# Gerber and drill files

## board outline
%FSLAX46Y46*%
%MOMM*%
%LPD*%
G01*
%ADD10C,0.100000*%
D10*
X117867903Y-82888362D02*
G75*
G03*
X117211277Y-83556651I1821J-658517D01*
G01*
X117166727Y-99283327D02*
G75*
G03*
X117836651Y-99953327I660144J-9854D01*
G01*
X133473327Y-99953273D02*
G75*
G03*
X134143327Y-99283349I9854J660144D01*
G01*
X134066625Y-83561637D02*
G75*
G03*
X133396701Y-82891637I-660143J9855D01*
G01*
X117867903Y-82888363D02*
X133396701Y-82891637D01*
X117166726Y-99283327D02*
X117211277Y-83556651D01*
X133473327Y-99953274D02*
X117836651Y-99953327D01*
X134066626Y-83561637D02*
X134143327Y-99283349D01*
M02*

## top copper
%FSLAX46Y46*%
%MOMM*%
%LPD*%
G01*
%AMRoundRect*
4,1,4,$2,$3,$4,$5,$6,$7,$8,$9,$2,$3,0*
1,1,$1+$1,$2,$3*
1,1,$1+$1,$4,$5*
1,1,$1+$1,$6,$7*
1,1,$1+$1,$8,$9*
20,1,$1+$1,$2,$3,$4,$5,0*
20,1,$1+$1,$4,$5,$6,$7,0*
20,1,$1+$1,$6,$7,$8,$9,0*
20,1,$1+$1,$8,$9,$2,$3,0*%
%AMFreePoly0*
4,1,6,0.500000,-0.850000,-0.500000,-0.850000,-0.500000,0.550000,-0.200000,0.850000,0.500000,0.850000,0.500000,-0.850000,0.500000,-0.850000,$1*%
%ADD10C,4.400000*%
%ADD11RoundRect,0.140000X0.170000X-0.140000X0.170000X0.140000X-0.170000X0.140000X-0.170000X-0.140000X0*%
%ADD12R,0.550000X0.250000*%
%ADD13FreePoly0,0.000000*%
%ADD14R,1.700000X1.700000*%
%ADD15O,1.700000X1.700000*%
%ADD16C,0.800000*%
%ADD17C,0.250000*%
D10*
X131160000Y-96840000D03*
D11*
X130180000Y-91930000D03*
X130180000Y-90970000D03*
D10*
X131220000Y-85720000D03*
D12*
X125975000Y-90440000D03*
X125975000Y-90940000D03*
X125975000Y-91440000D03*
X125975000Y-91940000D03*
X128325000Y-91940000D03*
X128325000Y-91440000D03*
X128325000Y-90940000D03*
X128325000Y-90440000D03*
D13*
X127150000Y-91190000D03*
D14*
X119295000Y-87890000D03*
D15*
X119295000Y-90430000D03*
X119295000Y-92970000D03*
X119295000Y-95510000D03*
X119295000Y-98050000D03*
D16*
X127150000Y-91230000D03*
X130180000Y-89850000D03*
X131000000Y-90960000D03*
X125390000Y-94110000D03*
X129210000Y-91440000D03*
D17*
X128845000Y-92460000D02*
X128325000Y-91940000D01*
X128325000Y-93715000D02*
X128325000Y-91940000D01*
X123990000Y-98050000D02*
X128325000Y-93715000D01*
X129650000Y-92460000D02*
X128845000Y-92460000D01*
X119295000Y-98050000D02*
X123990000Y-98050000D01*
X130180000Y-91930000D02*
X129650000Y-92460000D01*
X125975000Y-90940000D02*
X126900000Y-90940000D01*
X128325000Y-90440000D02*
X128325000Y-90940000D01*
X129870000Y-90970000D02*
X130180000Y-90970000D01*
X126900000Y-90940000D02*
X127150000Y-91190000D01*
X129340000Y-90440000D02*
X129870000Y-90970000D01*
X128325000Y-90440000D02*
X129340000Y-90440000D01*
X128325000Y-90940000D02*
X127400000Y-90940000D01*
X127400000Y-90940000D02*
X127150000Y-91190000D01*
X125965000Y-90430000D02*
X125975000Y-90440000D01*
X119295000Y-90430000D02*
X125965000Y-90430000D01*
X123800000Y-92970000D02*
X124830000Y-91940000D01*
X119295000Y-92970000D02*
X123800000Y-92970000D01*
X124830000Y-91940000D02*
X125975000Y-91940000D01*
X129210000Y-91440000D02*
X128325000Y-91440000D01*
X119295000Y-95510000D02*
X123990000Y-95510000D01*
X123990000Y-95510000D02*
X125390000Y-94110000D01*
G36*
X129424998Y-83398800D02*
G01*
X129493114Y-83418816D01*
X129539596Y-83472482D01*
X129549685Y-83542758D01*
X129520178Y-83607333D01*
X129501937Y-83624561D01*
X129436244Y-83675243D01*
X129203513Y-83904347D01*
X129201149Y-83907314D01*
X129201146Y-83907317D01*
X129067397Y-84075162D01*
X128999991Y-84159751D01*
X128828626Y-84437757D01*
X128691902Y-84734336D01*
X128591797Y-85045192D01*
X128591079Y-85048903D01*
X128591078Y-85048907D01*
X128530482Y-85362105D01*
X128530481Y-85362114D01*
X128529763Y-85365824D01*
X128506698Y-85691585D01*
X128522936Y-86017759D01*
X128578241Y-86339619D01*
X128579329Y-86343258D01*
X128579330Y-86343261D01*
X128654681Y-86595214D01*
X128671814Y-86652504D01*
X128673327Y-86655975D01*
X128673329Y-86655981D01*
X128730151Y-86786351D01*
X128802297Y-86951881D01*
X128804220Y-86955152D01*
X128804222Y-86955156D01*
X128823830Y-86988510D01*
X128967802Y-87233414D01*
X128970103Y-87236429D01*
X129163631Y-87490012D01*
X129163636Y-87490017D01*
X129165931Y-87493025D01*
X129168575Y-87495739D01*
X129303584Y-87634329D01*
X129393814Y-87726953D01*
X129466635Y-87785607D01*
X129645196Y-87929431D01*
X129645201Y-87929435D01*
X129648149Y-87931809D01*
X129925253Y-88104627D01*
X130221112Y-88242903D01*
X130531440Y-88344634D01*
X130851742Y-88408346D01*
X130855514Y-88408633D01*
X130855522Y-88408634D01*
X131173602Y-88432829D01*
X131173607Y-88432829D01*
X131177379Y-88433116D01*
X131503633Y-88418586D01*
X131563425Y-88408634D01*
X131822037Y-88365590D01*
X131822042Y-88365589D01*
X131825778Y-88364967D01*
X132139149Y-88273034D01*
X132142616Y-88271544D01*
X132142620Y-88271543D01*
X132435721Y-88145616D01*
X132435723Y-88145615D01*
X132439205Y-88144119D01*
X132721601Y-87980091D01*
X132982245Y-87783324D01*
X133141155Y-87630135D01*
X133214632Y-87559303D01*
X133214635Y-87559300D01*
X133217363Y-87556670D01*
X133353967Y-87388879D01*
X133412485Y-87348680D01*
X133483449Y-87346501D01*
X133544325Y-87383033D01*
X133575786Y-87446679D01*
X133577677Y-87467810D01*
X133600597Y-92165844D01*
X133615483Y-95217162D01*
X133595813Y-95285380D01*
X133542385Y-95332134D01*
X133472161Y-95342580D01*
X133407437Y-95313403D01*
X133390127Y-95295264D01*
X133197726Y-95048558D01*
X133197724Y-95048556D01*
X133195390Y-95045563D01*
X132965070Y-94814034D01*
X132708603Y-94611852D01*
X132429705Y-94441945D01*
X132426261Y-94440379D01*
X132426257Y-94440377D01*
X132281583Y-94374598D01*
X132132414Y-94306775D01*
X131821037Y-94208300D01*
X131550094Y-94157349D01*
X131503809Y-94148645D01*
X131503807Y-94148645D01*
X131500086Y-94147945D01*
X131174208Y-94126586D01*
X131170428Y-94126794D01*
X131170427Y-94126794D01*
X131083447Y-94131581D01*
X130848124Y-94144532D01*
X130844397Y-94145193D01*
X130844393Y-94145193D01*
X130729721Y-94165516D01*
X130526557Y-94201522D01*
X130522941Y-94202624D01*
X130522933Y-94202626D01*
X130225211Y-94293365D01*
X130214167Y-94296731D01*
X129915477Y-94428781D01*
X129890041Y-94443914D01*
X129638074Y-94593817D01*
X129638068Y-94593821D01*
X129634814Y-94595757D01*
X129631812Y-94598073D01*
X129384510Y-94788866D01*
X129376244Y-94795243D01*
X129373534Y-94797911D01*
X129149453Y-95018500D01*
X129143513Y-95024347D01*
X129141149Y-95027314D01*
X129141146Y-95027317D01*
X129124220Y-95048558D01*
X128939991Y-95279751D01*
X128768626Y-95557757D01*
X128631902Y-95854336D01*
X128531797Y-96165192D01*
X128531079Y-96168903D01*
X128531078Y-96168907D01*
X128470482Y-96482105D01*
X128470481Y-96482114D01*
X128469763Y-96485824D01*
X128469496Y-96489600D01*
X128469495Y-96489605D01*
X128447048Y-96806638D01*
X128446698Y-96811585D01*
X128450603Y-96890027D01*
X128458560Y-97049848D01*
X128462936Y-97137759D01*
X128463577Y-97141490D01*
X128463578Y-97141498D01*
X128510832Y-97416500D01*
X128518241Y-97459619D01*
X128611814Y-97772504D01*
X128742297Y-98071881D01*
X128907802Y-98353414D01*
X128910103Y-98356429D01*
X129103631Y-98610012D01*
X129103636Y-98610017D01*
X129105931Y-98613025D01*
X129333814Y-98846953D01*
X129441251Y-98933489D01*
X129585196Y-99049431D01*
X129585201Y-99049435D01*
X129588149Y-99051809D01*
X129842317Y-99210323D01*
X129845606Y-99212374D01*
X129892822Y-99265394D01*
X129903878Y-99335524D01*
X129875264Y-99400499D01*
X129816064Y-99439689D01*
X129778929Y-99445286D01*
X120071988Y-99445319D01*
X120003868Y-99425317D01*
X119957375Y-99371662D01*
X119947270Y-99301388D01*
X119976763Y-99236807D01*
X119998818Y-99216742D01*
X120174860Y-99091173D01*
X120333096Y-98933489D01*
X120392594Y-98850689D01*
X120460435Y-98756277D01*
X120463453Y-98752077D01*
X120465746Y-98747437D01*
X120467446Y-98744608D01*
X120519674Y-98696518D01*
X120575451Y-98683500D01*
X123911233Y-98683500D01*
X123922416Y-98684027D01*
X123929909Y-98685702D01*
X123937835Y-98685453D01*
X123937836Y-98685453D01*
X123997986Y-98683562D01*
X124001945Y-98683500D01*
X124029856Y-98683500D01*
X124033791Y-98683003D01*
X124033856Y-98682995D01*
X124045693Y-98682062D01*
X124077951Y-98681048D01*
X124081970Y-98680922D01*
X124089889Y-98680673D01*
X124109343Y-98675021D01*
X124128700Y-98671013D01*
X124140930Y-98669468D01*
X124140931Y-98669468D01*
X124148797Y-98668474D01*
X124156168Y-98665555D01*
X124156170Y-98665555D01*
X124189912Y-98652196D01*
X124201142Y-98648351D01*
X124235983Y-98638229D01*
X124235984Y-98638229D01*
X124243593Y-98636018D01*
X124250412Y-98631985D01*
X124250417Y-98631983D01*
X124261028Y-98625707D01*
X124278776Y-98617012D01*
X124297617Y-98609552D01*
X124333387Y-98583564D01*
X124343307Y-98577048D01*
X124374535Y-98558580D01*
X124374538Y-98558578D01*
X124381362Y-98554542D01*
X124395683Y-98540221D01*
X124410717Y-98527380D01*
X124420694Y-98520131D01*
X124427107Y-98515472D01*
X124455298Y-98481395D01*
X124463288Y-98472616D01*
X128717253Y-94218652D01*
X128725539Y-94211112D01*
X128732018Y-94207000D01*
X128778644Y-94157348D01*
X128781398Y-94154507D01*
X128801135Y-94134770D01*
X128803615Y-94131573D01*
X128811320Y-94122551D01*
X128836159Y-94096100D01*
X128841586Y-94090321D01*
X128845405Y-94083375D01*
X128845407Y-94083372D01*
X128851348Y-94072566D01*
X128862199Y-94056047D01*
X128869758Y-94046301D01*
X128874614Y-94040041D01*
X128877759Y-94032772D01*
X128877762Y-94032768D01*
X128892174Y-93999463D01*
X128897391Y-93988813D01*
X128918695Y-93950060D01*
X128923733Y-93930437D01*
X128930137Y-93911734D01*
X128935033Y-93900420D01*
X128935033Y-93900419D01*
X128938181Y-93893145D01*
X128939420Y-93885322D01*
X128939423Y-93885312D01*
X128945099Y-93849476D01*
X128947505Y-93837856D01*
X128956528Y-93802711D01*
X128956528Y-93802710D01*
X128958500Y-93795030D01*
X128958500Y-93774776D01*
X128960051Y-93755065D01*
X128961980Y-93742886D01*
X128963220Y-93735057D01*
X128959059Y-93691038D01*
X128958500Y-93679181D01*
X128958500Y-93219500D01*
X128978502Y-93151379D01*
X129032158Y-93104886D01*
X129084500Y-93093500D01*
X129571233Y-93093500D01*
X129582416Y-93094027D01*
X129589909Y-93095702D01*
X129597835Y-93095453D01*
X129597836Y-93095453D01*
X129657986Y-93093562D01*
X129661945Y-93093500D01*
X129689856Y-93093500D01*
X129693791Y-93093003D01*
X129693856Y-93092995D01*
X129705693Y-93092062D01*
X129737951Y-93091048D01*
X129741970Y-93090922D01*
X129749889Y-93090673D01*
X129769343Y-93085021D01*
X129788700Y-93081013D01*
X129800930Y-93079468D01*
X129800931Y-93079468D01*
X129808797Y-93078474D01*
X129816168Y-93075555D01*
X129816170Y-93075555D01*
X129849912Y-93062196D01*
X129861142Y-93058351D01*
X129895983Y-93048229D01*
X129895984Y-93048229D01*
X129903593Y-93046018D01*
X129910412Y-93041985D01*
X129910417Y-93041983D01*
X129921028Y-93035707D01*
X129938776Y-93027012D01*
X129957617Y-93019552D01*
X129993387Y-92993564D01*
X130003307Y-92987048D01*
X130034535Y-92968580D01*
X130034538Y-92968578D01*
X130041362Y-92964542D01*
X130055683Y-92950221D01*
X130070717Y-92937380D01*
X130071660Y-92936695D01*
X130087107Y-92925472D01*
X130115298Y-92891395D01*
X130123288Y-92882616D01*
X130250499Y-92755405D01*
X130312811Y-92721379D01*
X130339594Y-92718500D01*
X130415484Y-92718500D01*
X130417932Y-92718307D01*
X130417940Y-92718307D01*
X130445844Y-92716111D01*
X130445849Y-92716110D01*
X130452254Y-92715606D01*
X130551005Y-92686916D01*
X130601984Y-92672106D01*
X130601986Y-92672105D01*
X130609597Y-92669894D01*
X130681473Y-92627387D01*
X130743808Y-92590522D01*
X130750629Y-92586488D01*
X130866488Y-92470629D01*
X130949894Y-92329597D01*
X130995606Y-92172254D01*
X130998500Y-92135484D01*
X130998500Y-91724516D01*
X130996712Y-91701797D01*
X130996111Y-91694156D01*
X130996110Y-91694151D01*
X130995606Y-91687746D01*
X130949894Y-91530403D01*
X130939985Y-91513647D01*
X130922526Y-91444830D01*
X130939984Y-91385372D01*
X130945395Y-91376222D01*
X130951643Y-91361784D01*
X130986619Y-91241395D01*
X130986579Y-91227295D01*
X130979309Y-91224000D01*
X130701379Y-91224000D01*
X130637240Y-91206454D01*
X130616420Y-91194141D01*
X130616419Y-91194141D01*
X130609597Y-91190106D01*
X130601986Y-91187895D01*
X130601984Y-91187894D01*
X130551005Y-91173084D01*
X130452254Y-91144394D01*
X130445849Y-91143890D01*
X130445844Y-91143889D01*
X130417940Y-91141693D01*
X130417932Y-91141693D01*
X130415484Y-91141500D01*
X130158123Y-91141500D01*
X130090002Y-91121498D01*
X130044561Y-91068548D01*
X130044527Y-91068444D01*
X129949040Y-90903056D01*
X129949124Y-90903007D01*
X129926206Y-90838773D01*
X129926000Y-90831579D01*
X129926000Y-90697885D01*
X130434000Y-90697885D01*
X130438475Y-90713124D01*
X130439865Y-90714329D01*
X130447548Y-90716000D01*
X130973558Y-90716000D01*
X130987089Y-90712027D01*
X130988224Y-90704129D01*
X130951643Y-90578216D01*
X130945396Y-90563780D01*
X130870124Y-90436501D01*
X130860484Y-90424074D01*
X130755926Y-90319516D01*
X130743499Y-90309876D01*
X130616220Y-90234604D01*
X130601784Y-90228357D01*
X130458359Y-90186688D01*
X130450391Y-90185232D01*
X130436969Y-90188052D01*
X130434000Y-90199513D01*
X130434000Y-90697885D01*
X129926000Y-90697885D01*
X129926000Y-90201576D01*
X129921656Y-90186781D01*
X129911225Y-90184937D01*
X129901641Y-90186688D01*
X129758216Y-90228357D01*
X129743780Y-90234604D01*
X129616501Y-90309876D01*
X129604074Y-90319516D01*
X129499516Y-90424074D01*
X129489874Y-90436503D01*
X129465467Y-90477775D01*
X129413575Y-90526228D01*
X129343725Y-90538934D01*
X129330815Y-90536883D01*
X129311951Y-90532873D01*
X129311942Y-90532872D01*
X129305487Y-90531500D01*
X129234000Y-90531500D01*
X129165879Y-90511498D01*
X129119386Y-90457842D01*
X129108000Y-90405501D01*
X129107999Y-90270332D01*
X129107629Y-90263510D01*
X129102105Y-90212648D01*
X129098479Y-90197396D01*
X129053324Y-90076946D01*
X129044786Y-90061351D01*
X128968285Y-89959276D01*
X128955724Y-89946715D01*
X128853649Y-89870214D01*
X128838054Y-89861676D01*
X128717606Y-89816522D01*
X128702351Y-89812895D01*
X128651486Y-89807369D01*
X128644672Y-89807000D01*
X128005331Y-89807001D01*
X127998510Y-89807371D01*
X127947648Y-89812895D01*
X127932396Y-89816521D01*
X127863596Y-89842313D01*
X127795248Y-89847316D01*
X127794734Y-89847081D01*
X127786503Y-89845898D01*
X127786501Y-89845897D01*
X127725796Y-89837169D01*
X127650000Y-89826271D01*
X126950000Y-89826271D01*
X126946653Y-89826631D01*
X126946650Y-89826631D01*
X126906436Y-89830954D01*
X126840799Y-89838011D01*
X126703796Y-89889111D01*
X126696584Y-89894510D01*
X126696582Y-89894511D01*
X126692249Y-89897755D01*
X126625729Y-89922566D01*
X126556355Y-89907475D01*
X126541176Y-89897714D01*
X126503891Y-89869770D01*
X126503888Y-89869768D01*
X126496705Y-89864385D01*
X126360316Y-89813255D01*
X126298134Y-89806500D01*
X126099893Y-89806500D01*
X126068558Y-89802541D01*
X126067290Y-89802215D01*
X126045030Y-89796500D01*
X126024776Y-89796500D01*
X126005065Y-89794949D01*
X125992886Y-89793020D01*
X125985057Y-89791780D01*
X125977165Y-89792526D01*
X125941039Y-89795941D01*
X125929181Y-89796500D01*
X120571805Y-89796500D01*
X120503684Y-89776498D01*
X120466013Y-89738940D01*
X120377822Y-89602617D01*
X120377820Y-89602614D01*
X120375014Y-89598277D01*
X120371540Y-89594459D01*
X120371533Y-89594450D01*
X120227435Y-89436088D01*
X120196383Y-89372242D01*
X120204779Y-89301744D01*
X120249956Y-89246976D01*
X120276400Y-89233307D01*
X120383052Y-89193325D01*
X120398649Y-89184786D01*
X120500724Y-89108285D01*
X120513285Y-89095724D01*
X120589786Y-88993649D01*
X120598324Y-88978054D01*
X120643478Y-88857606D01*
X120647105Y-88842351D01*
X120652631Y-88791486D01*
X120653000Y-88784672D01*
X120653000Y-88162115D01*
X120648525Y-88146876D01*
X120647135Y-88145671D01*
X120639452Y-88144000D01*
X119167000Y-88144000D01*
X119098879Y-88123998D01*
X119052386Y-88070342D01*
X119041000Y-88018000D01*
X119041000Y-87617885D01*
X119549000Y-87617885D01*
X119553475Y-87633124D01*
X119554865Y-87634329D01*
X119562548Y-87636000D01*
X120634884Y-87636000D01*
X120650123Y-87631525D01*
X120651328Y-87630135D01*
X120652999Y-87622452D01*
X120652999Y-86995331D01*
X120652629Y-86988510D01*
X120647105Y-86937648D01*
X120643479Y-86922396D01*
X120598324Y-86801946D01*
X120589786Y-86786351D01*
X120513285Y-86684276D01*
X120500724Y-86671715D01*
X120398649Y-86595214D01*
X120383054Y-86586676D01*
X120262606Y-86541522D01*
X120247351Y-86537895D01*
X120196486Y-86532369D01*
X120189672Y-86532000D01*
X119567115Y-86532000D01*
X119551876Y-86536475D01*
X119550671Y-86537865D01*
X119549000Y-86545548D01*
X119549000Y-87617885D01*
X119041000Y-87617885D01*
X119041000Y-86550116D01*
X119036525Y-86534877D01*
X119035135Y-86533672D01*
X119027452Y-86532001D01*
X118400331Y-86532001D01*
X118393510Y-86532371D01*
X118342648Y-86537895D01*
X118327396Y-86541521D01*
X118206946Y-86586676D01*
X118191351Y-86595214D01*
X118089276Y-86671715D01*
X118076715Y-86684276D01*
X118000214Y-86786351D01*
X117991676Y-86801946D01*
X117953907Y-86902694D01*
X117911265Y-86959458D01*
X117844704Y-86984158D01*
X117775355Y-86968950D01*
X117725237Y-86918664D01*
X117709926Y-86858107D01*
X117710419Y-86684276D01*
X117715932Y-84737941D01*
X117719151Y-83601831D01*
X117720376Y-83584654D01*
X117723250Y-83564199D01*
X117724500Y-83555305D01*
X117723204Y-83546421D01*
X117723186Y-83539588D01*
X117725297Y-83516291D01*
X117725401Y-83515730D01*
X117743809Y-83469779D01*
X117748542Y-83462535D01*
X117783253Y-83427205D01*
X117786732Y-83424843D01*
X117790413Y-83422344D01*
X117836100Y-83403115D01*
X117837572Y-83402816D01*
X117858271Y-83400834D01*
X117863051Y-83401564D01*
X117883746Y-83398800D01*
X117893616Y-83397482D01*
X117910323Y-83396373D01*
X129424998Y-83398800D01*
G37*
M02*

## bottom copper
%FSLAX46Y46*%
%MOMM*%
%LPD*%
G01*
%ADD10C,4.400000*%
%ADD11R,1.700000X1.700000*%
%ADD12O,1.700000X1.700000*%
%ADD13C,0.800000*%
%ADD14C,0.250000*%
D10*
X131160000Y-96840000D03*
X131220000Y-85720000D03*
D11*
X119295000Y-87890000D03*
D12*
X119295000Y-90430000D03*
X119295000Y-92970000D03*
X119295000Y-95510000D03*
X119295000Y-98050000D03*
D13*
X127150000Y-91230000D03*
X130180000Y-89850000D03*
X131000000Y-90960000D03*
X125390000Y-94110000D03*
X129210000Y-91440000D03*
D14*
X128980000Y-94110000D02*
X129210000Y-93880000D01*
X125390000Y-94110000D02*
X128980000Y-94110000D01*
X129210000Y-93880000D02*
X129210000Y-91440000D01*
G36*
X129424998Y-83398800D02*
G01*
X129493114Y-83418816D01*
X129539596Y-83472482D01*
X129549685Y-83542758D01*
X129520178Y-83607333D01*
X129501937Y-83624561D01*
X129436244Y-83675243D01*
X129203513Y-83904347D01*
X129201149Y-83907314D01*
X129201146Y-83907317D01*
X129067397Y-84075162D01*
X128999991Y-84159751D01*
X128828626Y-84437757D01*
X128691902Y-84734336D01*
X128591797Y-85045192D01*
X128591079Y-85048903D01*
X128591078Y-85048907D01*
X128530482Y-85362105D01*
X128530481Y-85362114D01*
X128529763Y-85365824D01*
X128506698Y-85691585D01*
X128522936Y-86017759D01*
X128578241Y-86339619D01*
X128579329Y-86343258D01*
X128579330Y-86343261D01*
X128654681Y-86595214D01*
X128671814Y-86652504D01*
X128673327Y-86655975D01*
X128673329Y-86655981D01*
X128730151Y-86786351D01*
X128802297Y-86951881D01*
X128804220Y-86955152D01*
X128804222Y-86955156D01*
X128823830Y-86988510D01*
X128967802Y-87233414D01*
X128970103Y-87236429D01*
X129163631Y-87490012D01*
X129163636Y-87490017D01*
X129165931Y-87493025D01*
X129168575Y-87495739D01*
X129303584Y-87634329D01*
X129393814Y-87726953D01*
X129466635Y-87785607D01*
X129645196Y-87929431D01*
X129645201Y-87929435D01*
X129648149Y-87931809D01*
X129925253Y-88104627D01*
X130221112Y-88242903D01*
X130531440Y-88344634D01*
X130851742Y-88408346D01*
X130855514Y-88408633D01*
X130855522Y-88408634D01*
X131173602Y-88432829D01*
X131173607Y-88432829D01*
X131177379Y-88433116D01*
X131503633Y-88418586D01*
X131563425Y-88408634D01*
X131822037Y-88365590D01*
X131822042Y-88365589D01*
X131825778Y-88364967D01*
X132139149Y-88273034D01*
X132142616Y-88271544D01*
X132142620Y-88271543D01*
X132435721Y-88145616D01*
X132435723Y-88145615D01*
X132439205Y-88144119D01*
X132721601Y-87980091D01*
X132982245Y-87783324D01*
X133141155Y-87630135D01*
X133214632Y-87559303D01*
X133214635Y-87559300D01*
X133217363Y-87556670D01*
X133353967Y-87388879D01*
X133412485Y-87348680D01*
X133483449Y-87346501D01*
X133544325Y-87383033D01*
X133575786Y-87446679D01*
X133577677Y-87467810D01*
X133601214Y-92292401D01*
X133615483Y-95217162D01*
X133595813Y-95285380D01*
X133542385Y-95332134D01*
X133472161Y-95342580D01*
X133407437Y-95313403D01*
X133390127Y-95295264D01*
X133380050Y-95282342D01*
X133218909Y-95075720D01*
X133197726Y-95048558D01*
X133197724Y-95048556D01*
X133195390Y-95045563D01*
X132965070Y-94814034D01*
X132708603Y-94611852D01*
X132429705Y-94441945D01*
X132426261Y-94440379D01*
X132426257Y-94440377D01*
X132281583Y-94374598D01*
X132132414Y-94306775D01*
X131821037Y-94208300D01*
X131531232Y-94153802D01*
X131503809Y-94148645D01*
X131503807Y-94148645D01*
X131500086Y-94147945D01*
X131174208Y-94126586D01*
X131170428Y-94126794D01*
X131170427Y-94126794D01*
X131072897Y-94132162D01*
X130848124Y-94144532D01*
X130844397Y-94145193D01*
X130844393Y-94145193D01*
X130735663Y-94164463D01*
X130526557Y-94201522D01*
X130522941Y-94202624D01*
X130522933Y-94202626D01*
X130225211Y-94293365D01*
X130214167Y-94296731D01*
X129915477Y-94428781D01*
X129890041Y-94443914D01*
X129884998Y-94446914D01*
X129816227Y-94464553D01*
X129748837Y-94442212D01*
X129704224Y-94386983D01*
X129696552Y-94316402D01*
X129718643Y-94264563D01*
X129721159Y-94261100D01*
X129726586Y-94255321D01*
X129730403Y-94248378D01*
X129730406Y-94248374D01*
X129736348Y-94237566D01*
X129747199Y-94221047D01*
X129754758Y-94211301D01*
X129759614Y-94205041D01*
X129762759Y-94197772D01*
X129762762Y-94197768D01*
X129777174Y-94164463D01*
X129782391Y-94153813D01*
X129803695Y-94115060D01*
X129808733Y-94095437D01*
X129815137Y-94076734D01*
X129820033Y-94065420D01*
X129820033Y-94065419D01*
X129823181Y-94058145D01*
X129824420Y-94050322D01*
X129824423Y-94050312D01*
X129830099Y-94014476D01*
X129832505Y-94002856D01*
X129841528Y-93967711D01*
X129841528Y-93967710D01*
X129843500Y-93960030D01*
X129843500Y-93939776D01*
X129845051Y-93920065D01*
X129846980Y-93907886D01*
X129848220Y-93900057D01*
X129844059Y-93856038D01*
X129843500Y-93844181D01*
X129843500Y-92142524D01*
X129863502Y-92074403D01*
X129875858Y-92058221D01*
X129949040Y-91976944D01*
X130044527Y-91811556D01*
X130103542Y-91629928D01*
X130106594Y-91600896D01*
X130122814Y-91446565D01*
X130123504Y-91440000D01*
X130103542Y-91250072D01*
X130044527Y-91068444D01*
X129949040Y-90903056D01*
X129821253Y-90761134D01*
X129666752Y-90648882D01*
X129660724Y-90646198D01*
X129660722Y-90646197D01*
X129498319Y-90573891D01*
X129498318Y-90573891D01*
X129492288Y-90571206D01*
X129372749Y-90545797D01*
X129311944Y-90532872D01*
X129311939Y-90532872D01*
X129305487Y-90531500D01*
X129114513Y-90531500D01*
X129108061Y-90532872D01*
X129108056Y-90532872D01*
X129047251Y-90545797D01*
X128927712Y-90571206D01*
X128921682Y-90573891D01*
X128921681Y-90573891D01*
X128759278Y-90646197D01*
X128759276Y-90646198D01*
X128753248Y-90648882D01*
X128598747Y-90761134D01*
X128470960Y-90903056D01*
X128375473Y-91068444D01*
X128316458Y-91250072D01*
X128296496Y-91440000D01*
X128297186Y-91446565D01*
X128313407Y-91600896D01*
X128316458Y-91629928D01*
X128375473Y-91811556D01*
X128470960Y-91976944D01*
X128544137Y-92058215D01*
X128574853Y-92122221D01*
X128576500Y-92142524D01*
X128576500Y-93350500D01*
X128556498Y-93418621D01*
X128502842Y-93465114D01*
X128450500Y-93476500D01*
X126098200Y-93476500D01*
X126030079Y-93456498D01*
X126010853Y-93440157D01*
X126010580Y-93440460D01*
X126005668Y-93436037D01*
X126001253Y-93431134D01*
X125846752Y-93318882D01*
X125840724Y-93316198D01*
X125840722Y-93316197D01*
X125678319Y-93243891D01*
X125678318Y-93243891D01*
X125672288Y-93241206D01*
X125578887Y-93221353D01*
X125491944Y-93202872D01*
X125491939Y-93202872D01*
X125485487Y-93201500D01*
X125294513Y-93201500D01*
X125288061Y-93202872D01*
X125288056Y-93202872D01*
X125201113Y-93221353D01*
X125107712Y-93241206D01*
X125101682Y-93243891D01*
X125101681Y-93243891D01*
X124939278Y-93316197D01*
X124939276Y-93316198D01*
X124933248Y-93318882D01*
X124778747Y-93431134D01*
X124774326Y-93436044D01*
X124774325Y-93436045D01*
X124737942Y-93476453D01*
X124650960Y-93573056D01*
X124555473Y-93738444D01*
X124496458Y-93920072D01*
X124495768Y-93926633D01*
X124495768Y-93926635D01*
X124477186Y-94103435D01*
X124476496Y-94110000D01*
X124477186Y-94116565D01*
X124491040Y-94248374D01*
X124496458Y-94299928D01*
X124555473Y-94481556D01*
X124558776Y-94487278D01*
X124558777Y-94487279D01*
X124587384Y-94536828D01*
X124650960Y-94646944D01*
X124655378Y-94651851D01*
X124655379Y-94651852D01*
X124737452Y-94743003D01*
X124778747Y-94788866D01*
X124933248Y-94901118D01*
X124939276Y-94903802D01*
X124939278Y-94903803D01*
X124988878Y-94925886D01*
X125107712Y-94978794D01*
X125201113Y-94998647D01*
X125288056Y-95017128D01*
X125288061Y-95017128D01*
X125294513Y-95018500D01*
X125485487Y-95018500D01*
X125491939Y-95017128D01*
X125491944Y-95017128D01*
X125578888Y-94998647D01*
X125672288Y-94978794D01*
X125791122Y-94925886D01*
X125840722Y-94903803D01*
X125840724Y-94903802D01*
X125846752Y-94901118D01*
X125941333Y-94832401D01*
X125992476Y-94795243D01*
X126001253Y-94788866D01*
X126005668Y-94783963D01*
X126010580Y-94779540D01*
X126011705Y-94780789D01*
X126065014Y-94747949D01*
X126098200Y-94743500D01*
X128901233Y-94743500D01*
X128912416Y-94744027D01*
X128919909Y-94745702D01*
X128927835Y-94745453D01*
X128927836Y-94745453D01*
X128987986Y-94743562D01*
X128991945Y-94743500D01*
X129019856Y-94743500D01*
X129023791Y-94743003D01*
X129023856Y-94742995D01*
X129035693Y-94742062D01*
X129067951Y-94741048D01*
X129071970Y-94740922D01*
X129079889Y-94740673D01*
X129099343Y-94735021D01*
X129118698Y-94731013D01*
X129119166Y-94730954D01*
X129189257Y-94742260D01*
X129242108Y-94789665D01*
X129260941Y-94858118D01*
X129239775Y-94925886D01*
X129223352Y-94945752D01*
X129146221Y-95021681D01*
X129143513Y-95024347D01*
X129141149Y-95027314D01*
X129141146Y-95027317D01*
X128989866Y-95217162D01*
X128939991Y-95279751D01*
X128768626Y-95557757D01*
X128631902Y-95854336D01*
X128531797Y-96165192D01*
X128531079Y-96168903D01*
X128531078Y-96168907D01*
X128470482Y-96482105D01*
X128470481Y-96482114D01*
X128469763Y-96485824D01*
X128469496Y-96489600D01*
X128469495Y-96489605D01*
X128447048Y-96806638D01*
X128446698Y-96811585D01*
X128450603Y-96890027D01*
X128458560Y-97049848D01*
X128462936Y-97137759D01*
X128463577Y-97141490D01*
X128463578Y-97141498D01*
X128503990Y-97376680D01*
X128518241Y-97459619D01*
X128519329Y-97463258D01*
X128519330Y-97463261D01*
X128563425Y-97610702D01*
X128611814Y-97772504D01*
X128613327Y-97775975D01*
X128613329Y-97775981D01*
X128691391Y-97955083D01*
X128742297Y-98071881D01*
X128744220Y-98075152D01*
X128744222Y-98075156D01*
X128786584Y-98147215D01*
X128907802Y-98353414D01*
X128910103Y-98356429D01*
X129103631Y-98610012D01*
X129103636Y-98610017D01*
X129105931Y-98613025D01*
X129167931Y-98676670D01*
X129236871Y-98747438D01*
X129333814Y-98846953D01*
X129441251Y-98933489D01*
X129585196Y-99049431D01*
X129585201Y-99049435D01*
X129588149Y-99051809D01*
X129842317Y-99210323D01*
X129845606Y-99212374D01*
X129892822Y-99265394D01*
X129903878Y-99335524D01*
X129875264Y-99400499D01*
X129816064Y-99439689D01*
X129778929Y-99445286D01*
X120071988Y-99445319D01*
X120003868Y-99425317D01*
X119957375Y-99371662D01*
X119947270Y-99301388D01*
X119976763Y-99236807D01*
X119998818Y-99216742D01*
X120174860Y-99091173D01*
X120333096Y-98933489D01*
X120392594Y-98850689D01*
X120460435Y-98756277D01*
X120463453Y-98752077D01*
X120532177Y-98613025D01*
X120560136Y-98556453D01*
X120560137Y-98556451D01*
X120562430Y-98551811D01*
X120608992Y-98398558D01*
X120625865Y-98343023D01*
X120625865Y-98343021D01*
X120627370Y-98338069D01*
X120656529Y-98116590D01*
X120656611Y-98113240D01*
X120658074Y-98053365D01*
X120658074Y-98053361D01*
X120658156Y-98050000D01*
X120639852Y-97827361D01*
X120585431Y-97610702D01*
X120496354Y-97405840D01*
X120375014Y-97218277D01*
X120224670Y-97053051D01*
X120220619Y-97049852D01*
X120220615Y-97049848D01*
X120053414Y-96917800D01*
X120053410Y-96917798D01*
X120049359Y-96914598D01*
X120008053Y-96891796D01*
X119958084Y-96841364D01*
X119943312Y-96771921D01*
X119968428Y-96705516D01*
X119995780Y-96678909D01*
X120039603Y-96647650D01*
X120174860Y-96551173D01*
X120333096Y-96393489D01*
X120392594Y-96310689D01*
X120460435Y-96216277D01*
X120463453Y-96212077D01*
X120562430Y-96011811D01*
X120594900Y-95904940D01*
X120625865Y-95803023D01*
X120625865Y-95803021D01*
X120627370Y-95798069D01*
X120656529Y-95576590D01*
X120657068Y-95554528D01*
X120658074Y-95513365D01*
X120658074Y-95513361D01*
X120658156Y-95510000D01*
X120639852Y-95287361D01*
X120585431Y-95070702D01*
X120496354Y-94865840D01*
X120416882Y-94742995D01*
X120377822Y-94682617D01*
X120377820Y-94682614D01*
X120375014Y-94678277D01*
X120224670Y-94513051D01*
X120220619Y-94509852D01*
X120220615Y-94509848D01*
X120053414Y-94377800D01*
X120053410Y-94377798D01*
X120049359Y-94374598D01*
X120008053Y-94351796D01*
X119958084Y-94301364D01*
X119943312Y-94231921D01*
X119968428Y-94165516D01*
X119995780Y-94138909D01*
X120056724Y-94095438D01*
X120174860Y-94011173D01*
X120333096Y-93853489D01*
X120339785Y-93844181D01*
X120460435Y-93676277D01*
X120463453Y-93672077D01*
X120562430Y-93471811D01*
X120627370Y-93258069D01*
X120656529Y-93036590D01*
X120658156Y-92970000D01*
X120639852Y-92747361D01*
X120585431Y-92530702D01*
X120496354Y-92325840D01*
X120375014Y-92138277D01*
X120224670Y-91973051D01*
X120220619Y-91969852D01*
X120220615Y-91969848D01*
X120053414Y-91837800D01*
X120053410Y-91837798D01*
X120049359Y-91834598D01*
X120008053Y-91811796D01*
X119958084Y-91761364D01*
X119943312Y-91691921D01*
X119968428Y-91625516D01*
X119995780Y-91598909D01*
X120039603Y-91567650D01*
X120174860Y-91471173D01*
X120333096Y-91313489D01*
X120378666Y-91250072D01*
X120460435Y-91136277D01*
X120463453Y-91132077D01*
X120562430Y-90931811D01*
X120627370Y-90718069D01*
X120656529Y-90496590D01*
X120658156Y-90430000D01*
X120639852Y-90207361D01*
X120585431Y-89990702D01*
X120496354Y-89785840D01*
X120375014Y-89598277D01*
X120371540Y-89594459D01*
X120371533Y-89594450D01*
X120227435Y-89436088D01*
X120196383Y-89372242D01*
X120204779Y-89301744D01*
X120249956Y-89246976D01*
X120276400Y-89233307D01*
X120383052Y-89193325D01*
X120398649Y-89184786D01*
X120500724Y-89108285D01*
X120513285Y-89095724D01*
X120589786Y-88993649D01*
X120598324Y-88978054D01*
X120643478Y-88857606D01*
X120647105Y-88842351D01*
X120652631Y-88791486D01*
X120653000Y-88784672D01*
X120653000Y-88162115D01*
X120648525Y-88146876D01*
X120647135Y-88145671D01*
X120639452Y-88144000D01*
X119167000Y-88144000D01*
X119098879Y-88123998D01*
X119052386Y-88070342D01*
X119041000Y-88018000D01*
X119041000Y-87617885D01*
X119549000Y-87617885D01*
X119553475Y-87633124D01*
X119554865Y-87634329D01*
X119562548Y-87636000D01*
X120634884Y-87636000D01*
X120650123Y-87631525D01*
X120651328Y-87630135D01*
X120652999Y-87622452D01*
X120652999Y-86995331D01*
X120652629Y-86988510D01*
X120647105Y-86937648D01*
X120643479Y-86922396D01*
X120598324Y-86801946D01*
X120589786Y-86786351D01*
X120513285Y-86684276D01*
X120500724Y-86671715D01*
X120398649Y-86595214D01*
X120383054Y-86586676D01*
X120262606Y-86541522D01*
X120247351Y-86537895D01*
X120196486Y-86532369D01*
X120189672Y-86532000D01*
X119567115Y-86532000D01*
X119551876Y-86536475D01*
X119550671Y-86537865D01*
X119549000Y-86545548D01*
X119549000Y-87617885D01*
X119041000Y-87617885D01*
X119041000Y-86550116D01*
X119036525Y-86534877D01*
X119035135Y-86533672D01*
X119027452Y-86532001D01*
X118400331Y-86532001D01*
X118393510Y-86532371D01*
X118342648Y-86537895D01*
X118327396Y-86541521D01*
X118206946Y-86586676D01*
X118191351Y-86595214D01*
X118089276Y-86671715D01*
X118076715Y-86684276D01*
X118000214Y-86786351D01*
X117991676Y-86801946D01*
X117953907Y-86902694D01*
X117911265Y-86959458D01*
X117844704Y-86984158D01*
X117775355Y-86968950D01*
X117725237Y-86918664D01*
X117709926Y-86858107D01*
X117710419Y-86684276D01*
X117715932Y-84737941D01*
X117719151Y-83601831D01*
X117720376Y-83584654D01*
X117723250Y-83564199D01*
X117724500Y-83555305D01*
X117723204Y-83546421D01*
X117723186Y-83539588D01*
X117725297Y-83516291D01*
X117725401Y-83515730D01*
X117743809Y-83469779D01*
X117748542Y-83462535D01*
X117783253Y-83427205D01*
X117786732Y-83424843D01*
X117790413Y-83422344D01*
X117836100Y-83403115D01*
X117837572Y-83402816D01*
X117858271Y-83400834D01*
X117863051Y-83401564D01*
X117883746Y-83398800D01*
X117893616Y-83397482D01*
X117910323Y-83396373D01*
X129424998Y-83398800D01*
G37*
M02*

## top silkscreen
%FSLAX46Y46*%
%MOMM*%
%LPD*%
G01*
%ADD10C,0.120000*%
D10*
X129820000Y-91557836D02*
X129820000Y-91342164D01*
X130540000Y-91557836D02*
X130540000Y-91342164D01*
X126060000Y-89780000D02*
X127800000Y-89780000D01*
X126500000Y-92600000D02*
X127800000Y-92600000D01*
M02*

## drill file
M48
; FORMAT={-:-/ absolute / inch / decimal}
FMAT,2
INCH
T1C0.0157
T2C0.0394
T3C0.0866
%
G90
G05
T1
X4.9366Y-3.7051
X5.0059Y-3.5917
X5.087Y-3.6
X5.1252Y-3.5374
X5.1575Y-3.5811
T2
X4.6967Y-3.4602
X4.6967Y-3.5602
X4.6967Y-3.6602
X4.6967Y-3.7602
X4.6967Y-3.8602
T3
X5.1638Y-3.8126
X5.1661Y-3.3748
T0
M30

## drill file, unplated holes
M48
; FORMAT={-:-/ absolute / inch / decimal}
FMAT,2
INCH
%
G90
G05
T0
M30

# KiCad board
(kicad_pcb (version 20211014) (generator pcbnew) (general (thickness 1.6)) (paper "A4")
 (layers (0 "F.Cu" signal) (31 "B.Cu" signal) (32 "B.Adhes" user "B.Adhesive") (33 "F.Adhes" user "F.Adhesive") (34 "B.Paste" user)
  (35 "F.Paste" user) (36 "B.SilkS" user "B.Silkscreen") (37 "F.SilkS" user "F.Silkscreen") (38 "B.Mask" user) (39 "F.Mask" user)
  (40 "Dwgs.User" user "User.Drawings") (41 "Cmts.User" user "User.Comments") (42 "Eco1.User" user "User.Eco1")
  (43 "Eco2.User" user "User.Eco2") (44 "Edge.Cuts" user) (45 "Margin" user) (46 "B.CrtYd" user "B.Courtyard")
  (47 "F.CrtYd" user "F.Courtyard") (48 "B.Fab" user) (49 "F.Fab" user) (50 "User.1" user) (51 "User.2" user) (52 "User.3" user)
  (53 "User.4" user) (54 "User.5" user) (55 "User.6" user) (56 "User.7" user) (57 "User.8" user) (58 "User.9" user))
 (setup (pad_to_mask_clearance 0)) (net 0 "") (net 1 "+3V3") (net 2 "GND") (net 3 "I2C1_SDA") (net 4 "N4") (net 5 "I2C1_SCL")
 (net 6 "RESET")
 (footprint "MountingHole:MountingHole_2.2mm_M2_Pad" (layer "F.Cu") (at 131.16 96.84)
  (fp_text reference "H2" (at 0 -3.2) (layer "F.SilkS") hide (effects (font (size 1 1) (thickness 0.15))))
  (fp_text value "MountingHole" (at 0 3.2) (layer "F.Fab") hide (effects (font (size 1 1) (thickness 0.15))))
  (pad "1" thru_hole circle (at 0 0) (size 4.4 4.4) (drill 2.2) (layers *.Cu *.Mask)))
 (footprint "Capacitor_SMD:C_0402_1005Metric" (layer "F.Cu") (at 130.18 91.45 90)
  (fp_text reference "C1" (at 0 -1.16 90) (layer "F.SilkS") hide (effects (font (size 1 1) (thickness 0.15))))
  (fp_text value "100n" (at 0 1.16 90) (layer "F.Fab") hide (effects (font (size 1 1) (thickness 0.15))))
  (fp_line (start -0.107836 -0.36) (end 0.107836 -0.36) (layer "F.SilkS") (width 0.12))
  (fp_line (start -0.107836 0.36) (end 0.107836 0.36) (layer "F.SilkS") (width 0.12))
  (pad "1" smd roundrect (at -0.48 0 90) (size 0.56 0.62) (layers "F.Cu" "F.Paste" "F.Mask") (roundrect_rratio 0.25) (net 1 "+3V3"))
  (pad "2" smd roundrect (at 0.48 0 90) (size 0.56 0.62) (layers "F.Cu" "F.Paste" "F.Mask") (roundrect_rratio 0.25) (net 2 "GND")))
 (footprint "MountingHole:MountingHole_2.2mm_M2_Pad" (layer "F.Cu") (at 131.22 85.72)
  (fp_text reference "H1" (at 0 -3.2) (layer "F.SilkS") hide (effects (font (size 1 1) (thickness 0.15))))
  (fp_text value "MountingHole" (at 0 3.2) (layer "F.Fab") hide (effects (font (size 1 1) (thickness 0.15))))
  (pad "1" thru_hole circle (at 0 0) (size 4.4 4.4) (drill 2.2) (layers *.Cu *.Mask)))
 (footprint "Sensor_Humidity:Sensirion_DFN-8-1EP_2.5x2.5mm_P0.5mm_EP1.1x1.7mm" (layer "F.Cu") (at 127.15 91.19)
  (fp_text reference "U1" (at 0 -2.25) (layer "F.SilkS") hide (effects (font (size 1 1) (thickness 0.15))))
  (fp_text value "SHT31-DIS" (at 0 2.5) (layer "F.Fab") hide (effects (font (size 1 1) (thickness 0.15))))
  (fp_line (start -1.09 -1.41) (end 0.65 -1.41) (layer "F.SilkS") (width 0.12))
  (fp_line (start -0.65 1.41) (end 0.65 1.41) (layer "F.SilkS") (width 0.12))
  (pad "" smd custom (at 0 0) (size 0.9 0.9) (layers "F.Paste") (zone_connect 0) (options (clearance outline) (anchor rect)) (primitives))
  (pad "1" smd rect (at -1.175 -0.75) (size 0.55 0.25) (layers "F.Cu" "F.Paste" "F.Mask") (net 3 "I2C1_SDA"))
  (pad "2" smd rect (at -1.175 -0.25) (size 0.55 0.25) (layers "F.Cu" "F.Paste" "F.Mask") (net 2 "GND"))
  (pad "3" smd rect (at -1.175 0.25) (size 0.55 0.25) (layers "F.Cu" "F.Paste" "F.Mask") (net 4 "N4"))
  (pad "4" smd rect (at -1.175 0.75 180) (size 0.55 0.25) (layers "F.Cu" "F.Paste" "F.Mask") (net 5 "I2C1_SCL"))
  (pad "5" smd rect (at 1.175 0.75) (size 0.55 0.25) (layers "F.Cu" "F.Paste" "F.Mask") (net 1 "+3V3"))
  (pad "6" smd rect (at 1.175 0.25) (size 0.55 0.25) (layers "F.Cu" "F.Paste" "F.Mask") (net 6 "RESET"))
  (pad "7" smd rect (at 1.175 -0.25) (size 0.55 0.25) (layers "F.Cu" "F.Paste" "F.Mask") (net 2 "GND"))
  (pad "8" smd rect (at 1.175 -0.75) (size 0.55 0.25) (layers "F.Cu" "F.Paste" "F.Mask") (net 2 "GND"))
  (pad "9" smd custom (at 0 0) (size 1 1) (layers "F.Cu" "F.Mask") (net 2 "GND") (zone_connect 0)
   (options (clearance outline) (anchor circle)) (primitives)))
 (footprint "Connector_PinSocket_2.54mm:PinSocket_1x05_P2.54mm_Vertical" (layer "B.Cu") (at 119.295 87.89 180)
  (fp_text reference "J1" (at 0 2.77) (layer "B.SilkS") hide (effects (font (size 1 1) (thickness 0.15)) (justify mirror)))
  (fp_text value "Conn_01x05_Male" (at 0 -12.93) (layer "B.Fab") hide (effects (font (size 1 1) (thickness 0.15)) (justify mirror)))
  (pad "1" thru_hole rect (at 0 0 180) (size 1.7 1.7) (drill 1) (layers *.Cu *.Mask) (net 2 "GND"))
  (pad "2" thru_hole oval (at 0 -2.54 180) (size 1.7 1.7) (drill 1) (layers *.Cu *.Mask) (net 3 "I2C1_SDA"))
  (pad "3" thru_hole oval (at 0 -5.08 180) (size 1.7 1.7) (drill 1) (layers *.Cu *.Mask) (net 5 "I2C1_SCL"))
  (pad "4" thru_hole oval (at 0 -7.62 180) (size 1.7 1.7) (drill 1) (layers *.Cu *.Mask) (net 6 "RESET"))
  (pad "5" thru_hole oval (at 0 -10.16 180) (size 1.7 1.7) (drill 1) (layers *.Cu *.Mask) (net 1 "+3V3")))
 (gr_line (start 133.473327 99.953274) (end 117.836651 99.953327) (layer "Edge.Cuts") (width 0.1))
 (gr_arc (start 134.143327 99.283349) (mid 133.95 99.76) (end 133.473327 99.953274) (layer "Edge.Cuts") (width 0.1))
 (gr_arc (start 117.836651 99.953327) (mid 117.36 99.76) (end 117.166726 99.283327) (layer "Edge.Cuts") (width 0.1))
 (gr_line (start 134.066626 83.561637) (end 134.143327 99.283349) (layer "Edge.Cuts") (width 0.1))
 (gr_line (start 117.166726 99.283327) (end 117.211277 83.556651) (layer "Edge.Cuts") (width 0.1))
 (gr_line (start 117.867903 82.888363) (end 133.396701 82.891637) (layer "Edge.Cuts") (width 0.1))
 (gr_arc (start 117.211277 83.556651) (mid 117.4 83.085352) (end 117.867903 82.888363) (layer "Edge.Cuts") (width 0.1))
 (gr_arc (start 133.396701 82.891637) (mid 133.873352 83.084964) (end 134.066626 83.561637) (layer "Edge.Cuts") (width 0.1))
 (segment (start 128.845 92.46) (end 128.325 91.94) (width 0.25) (layer "F.Cu") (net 1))
 (segment (start 128.325 93.715) (end 128.325 91.94) (width 0.25) (layer "F.Cu") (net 1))
 (segment (start 123.99 98.05) (end 128.325 93.715) (width 0.25) (layer "F.Cu") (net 1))
 (segment (start 129.65 92.46) (end 128.845 92.46) (width 0.25) (layer "F.Cu") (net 1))
 (segment (start 119.295 98.05) (end 123.99 98.05) (width 0.25) (layer "F.Cu") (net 1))
 (segment (start 130.18 91.93) (end 129.65 92.46) (width 0.25) (layer "F.Cu") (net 1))
 (segment (start 125.975 90.94) (end 126.9 90.94) (width 0.25) (layer "F.Cu") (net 2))
 (segment (start 128.325 90.44) (end 128.325 90.94) (width 0.25) (layer "F.Cu") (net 2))
 (segment (start 129.87 90.97) (end 130.18 90.97) (width 0.25) (layer "F.Cu") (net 2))
 (segment (start 126.9 90.94) (end 127.15 91.19) (width 0.25) (layer "F.Cu") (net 2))
 (segment (start 129.34 90.44) (end 129.87 90.97) (width 0.25) (layer "F.Cu") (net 2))
 (segment (start 128.325 90.44) (end 129.34 90.44) (width 0.25) (layer "F.Cu") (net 2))
 (segment (start 128.325 90.94) (end 127.4 90.94) (width 0.25) (layer "F.Cu") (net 2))
 (segment (start 127.4 90.94) (end 127.15 91.19) (width 0.25) (layer "F.Cu") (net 2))
 (via (at 127.15 91.23) (size 0.8) (drill 0.4) (layers "F.Cu" "B.Cu") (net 2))
 (via (at 130.18 89.85) (size 0.8) (drill 0.4) (layers "F.Cu" "B.Cu") (free) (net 2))
 (via (at 131 90.96) (size 0.8) (drill 0.4) (layers "F.Cu" "B.Cu") (free) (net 2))
 (segment (start 125.965 90.43) (end 125.975 90.44) (width 0.25) (layer "F.Cu") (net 3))
 (segment (start 119.295 90.43) (end 125.965 90.43) (width 0.25) (layer "F.Cu") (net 3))
 (segment (start 123.8 92.97) (end 124.83 91.94) (width 0.25) (layer "F.Cu") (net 5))
 (segment (start 119.295 92.97) (end 123.8 92.97) (width 0.25) (layer "F.Cu") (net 5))
 (segment (start 124.83 91.94) (end 125.975 91.94) (width 0.25) (layer "F.Cu") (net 5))
 (segment (start 129.21 91.44) (end 128.325 91.44) (width 0.25) (layer "F.Cu") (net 6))
 (segment (start 119.295 95.51) (end 123.99 95.51) (width 0.25) (layer "F.Cu") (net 6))
 (segment (start 123.99 95.51) (end 125.39 94.11) (width 0.25) (layer "F.Cu") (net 6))
 (via (at 125.39 94.11) (size 0.8) (drill 0.4) (layers "F.Cu" "B.Cu") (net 6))
 (via (at 129.21 91.44) (size 0.8) (drill 0.4) (layers "F.Cu" "B.Cu") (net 6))
 (segment (start 128.98 94.11) (end 129.21 93.88) (width 0.25) (layer "B.Cu") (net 6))
 (segment (start 125.39 94.11) (end 128.98 94.11) (width 0.25) (layer "B.Cu") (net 6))
 (segment (start 129.21 93.88) (end 129.21 91.44) (width 0.25) (layer "B.Cu") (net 6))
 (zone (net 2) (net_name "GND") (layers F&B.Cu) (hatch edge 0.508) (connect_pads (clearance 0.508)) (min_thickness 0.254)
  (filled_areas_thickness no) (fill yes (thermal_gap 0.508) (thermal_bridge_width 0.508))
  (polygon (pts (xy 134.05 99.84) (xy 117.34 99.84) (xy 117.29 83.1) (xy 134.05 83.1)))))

